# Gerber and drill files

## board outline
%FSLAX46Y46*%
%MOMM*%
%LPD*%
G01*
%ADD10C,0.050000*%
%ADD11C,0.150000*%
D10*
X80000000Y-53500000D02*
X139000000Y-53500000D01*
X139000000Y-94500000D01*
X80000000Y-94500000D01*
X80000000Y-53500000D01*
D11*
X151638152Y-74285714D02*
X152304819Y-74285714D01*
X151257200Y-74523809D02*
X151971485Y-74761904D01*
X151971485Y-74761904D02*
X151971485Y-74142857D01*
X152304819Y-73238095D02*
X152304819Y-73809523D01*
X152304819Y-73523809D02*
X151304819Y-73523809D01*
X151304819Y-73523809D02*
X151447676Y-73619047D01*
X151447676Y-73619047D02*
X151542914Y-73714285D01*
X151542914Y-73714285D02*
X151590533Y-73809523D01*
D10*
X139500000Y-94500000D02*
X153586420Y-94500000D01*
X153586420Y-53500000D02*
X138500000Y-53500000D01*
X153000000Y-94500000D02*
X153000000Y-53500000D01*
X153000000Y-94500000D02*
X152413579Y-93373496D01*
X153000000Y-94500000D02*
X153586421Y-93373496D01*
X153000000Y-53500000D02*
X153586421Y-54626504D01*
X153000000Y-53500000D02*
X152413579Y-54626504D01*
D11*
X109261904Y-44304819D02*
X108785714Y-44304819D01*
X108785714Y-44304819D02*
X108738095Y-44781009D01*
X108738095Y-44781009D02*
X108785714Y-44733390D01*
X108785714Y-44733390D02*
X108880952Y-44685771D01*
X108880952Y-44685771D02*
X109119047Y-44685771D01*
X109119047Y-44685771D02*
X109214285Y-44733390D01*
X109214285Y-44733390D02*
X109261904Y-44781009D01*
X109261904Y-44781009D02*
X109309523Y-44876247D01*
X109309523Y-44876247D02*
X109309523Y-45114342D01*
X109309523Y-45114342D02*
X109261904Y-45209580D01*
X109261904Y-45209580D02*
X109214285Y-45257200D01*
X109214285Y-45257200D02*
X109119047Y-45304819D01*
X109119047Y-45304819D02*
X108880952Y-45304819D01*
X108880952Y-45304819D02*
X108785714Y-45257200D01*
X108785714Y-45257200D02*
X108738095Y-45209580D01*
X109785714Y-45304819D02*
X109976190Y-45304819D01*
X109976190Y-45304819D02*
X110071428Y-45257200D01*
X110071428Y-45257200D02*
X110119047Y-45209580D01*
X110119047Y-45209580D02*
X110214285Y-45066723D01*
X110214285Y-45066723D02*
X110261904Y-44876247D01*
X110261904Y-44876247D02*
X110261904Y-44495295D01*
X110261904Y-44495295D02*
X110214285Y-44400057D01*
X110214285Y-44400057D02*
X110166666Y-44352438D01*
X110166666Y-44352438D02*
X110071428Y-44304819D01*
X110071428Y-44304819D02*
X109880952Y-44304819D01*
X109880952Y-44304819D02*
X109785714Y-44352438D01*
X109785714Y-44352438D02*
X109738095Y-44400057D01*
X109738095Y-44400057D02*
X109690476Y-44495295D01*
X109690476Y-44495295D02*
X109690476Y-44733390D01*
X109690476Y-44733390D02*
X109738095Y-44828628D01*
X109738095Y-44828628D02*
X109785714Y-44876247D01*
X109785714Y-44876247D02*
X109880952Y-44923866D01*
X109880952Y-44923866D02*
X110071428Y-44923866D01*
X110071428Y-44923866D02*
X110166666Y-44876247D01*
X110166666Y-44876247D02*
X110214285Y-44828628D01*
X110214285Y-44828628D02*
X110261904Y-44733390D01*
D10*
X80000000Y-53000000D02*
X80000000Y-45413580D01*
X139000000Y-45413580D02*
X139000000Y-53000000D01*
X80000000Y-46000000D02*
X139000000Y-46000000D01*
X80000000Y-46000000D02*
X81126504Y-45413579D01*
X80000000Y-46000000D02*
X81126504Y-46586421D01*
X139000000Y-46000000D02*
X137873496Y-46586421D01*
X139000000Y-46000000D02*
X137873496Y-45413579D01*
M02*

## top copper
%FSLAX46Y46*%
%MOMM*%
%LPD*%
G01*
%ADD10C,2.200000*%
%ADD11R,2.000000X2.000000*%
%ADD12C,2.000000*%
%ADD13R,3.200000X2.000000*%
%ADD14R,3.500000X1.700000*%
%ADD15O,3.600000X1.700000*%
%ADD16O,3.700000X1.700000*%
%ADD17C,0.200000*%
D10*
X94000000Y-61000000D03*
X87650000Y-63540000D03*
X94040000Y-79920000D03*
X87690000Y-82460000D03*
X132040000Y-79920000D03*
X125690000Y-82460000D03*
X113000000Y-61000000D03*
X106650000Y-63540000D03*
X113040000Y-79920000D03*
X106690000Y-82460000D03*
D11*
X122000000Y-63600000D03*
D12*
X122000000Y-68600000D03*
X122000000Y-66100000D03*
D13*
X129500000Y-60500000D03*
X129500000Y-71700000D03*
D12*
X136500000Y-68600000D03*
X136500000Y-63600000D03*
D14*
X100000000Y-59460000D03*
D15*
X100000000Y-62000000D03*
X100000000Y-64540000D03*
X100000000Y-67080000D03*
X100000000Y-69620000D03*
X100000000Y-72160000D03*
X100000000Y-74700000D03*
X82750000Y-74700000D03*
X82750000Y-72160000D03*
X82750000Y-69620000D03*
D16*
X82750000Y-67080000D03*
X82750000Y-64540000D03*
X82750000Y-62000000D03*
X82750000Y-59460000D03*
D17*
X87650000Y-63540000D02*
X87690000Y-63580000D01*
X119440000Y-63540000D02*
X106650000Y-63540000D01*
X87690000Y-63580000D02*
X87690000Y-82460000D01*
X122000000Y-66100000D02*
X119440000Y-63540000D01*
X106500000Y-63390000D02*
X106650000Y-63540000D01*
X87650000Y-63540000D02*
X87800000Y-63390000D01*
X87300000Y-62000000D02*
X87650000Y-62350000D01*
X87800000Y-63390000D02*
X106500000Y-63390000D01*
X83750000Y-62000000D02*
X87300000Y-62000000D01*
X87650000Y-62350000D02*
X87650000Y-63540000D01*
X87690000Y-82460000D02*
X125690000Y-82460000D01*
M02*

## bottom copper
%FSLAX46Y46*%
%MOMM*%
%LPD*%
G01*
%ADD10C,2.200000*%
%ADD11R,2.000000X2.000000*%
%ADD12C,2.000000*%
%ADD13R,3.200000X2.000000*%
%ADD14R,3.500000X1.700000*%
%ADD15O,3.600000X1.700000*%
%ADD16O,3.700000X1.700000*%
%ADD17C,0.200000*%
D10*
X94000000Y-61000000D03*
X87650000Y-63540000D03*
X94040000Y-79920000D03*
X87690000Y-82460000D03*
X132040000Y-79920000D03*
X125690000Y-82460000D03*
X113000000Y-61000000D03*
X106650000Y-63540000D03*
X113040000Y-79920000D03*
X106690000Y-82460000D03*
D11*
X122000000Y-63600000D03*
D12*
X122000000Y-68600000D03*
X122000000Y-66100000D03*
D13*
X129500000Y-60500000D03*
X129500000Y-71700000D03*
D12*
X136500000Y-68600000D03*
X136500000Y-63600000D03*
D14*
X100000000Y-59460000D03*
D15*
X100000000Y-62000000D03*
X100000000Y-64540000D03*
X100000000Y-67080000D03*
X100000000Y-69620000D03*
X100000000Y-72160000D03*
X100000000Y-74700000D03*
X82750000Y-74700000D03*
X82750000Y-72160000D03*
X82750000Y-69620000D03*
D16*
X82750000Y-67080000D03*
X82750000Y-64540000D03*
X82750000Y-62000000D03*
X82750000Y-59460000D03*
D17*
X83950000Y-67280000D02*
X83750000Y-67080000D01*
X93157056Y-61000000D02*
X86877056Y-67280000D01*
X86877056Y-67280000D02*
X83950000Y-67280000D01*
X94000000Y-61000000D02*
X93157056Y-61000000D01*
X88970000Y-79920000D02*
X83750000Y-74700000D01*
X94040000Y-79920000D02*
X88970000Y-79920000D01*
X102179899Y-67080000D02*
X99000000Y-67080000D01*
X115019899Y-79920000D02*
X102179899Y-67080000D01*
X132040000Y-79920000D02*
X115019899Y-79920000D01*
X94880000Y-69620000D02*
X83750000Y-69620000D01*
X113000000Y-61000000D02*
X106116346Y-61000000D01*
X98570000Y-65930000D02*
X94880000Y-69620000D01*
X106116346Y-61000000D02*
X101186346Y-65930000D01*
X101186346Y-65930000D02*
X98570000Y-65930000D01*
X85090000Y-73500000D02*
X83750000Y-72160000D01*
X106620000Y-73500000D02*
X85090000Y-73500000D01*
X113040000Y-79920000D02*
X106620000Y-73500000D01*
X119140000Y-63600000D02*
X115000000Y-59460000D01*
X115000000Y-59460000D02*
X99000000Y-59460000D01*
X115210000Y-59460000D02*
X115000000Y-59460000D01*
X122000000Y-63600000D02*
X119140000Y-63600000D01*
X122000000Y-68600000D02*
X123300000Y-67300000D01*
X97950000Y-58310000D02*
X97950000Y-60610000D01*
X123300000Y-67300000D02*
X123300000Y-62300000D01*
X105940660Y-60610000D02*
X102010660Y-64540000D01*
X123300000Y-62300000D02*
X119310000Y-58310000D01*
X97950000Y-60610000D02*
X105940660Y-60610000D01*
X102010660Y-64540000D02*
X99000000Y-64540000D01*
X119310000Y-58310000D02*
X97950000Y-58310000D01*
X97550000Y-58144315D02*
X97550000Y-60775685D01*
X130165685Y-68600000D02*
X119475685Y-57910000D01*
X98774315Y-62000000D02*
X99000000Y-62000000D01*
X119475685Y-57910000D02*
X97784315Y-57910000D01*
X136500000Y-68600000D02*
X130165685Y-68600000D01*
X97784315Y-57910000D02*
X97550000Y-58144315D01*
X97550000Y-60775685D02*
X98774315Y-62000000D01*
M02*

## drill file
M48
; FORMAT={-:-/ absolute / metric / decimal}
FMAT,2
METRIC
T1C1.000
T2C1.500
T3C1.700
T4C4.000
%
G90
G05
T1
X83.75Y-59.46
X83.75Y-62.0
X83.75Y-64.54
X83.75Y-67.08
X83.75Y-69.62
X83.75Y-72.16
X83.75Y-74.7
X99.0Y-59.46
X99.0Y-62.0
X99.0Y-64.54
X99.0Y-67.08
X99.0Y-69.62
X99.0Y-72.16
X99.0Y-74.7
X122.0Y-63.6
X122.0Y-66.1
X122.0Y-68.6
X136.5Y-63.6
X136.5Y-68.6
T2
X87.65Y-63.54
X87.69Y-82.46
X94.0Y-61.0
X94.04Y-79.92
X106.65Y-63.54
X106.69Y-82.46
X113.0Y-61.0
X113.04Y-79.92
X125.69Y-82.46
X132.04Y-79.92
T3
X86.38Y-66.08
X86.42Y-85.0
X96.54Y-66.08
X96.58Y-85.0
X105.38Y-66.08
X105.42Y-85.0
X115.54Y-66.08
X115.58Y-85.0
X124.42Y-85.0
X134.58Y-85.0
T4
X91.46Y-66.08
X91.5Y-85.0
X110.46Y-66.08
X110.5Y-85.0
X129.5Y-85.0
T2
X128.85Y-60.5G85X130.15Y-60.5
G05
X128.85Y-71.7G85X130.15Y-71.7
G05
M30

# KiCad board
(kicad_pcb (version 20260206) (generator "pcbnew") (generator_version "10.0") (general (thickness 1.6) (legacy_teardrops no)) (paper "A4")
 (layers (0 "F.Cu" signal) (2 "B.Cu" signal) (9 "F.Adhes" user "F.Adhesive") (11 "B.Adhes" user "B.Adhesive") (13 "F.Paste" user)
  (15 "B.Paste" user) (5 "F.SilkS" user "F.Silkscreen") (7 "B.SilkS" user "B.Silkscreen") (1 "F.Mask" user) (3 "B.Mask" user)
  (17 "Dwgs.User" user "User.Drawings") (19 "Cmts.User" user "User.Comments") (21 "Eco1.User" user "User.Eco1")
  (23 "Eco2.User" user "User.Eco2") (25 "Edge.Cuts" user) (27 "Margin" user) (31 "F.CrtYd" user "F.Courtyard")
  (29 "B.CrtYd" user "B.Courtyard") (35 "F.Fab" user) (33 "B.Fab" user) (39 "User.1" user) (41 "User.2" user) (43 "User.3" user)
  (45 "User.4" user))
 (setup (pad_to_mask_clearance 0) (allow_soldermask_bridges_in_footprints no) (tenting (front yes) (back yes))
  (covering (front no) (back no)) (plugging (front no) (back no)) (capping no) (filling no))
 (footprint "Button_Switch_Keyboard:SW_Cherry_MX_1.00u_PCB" (layer "F.Cu") (at 94 61)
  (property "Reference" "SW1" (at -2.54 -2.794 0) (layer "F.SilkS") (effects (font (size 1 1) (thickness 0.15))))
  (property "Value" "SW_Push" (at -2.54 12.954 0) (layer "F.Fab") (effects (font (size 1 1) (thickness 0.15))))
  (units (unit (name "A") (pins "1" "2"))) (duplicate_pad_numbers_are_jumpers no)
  (pad "" np_thru_hole circle (at -7.62 5.08) (size 1.7 1.7) (drill 1.7) (layers "*.Cu" "*.Mask"))
  (pad "" np_thru_hole circle (at -2.54 5.08) (size 4 4) (drill 4) (layers "*.Cu" "*.Mask"))
  (pad "" np_thru_hole circle (at 2.54 5.08) (size 1.7 1.7) (drill 1.7) (layers "*.Cu" "*.Mask"))
  (pad "1" thru_hole circle (at 0 0) (size 2.2 2.2) (drill 1.5) (layers "*.Cu" "*.Mask") (remove_unused_layers no)
   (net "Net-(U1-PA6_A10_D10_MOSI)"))
  (pad "2" thru_hole circle (at -6.35 2.54) (size 2.2 2.2) (drill 1.5) (layers "*.Cu" "*.Mask") (remove_unused_layers no) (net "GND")))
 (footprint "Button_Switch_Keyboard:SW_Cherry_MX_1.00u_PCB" (layer "F.Cu") (at 94.04 79.92)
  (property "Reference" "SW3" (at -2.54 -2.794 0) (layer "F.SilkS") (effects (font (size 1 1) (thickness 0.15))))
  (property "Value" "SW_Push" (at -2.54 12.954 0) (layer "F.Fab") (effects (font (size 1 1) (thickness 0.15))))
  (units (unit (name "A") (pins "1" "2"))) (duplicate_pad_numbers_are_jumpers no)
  (pad "" np_thru_hole circle (at -7.62 5.08) (size 1.7 1.7) (drill 1.7) (layers "*.Cu" "*.Mask"))
  (pad "" np_thru_hole circle (at -2.54 5.08) (size 4 4) (drill 4) (layers "*.Cu" "*.Mask"))
  (pad "" np_thru_hole circle (at 2.54 5.08) (size 1.7 1.7) (drill 1.7) (layers "*.Cu" "*.Mask"))
  (pad "1" thru_hole circle (at 0 0) (size 2.2 2.2) (drill 1.5) (layers "*.Cu" "*.Mask") (remove_unused_layers no)
   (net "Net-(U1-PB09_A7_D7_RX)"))
  (pad "2" thru_hole circle (at -6.35 2.54) (size 2.2 2.2) (drill 1.5) (layers "*.Cu" "*.Mask") (remove_unused_layers no) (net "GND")))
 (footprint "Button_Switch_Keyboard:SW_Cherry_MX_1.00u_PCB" (layer "F.Cu") (at 132.04 79.92)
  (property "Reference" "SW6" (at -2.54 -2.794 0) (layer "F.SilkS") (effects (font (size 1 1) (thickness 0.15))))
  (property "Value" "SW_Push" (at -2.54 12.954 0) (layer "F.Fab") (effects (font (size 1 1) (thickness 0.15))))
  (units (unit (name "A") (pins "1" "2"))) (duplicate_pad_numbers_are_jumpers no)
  (pad "" np_thru_hole circle (at -7.62 5.08) (size 1.7 1.7) (drill 1.7) (layers "*.Cu" "*.Mask"))
  (pad "" np_thru_hole circle (at -2.54 5.08) (size 4 4) (drill 4) (layers "*.Cu" "*.Mask"))
  (pad "" np_thru_hole circle (at 2.54 5.08) (size 1.7 1.7) (drill 1.7) (layers "*.Cu" "*.Mask"))
  (pad "1" thru_hole circle (at 0 0) (size 2.2 2.2) (drill 1.5) (layers "*.Cu" "*.Mask") (remove_unused_layers no)
   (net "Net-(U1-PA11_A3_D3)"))
  (pad "2" thru_hole circle (at -6.35 2.54) (size 2.2 2.2) (drill 1.5) (layers "*.Cu" "*.Mask") (remove_unused_layers no) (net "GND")))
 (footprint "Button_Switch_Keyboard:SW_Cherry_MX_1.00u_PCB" (layer "F.Cu") (at 113 61)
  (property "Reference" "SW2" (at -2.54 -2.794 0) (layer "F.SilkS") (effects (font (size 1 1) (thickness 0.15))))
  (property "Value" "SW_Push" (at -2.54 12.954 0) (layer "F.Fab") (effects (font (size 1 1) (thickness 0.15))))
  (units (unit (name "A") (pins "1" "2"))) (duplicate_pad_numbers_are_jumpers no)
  (pad "" np_thru_hole circle (at -7.62 5.08) (size 1.7 1.7) (drill 1.7) (layers "*.Cu" "*.Mask"))
  (pad "" np_thru_hole circle (at -2.54 5.08) (size 4 4) (drill 4) (layers "*.Cu" "*.Mask"))
  (pad "" np_thru_hole circle (at 2.54 5.08) (size 1.7 1.7) (drill 1.7) (layers "*.Cu" "*.Mask"))
  (pad "1" thru_hole circle (at 0 0) (size 2.2 2.2) (drill 1.5) (layers "*.Cu" "*.Mask") (remove_unused_layers no)
   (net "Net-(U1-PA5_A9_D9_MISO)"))
  (pad "2" thru_hole circle (at -6.35 2.54) (size 2.2 2.2) (drill 1.5) (layers "*.Cu" "*.Mask") (remove_unused_layers no) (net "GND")))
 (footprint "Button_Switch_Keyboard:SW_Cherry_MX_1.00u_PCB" (layer "F.Cu") (at 113.04 79.92)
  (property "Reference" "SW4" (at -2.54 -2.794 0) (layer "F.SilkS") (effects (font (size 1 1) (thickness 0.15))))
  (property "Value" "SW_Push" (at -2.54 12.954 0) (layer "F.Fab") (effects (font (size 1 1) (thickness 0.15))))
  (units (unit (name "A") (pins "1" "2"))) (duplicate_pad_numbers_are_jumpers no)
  (pad "" np_thru_hole circle (at -7.62 5.08) (size 1.7 1.7) (drill 1.7) (layers "*.Cu" "*.Mask"))
  (pad "" np_thru_hole circle (at -2.54 5.08) (size 4 4) (drill 4) (layers "*.Cu" "*.Mask"))
  (pad "" np_thru_hole circle (at 2.54 5.08) (size 1.7 1.7) (drill 1.7) (layers "*.Cu" "*.Mask"))
  (pad "1" thru_hole circle (at 0 0) (size 2.2 2.2) (drill 1.5) (layers "*.Cu" "*.Mask") (remove_unused_layers no)
   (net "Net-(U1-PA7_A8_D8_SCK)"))
  (pad "2" thru_hole circle (at -6.35 2.54) (size 2.2 2.2) (drill 1.5) (layers "*.Cu" "*.Mask") (remove_unused_layers no) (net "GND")))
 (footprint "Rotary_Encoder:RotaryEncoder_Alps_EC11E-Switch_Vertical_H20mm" (layer "F.Cu") (at 122 63.6)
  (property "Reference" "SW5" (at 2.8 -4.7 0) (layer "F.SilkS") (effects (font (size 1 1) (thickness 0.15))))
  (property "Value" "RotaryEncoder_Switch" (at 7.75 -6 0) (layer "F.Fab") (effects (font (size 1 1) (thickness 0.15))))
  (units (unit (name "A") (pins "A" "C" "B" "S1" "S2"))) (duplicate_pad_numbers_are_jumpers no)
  (pad "A" thru_hole rect (at 0 0) (size 2 2) (drill 1) (layers "*.Cu" "*.Mask") (remove_unused_layers no) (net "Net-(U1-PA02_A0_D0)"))
  (pad "B" thru_hole circle (at 0 5) (size 2 2) (drill 1) (layers "*.Cu" "*.Mask") (remove_unused_layers no) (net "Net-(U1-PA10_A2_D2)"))
  (pad "C" thru_hole circle (at 0 2.5) (size 2 2) (drill 1) (layers "*.Cu" "*.Mask") (remove_unused_layers no) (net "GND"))
  (pad "MP" thru_hole rect (at 7.5 -3.1) (size 3.2 2) (drill oval 2.8 1.5) (layers "*.Cu" "*.Mask") (remove_unused_layers no))
  (pad "MP" thru_hole rect (at 7.5 8.1) (size 3.2 2) (drill oval 2.8 1.5) (layers "*.Cu" "*.Mask") (remove_unused_layers no))
  (pad "S1" thru_hole circle (at 14.5 5) (size 2 2) (drill 1) (layers "*.Cu" "*.Mask") (remove_unused_layers no) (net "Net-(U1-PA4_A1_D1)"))
  (pad "S2" thru_hole circle (at 14.5 0) (size 2 2) (drill 1) (layers "*.Cu" "*.Mask") (remove_unused_layers no)
   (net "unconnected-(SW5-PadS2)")))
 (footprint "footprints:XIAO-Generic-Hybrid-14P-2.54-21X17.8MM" (layer "B.Cu") (at 91.375 67.08 180)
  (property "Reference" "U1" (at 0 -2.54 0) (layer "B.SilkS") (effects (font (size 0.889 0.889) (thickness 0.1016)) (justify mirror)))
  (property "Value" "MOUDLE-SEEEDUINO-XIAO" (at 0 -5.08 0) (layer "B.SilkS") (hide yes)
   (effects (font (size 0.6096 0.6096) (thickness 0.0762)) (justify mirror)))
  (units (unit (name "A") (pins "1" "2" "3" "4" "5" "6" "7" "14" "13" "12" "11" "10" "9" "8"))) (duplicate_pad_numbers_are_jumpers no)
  (pad "1" thru_hole rect (at -7.625 7.62 180) (size 3.5 1.7) (drill 1 (offset -1 0)) (layers "*.Cu" "*.Mask") (remove_unused_layers no)
   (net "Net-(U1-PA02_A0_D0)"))
  (pad "2" thru_hole oval (at -7.625 5.08 180) (size 3.6 1.7) (drill 1 (offset -1 0)) (layers "*.Cu" "*.Mask") (remove_unused_layers no)
   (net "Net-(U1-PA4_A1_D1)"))
  (pad "3" thru_hole oval (at -7.625 2.54 180) (size 3.6 1.7) (drill 1 (offset -1 0)) (layers "*.Cu" "*.Mask") (remove_unused_layers no)
   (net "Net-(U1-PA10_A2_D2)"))
  (pad "4" thru_hole oval (at -7.625 0 180) (size 3.6 1.7) (drill 1 (offset -1 0)) (layers "*.Cu" "*.Mask") (remove_unused_layers no)
   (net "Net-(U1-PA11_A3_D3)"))
  (pad "5" thru_hole oval (at -7.625 -2.54 180) (size 3.6 1.7) (drill 1 (offset -1 0)) (layers "*.Cu" "*.Mask") (remove_unused_layers no)
   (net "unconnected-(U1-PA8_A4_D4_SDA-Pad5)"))
  (pad "6" thru_hole oval (at -7.625 -5.08) (size 3.6 1.7) (drill 1 (offset 1 0)) (layers "*.Cu" "*.Mask") (remove_unused_layers no)
   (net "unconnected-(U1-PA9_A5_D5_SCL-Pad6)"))
  (pad "7" thru_hole oval (at -7.625 -7.62 180) (size 3.6 1.7) (drill 1 (offset -1 0)) (layers "*.Cu" "*.Mask") (remove_unused_layers no)
   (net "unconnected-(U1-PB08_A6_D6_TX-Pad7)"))
  (pad "8" thru_hole oval (at 7.625 -7.62 180) (size 3.6 1.7) (drill 1 (offset 1 0)) (layers "*.Cu" "*.Mask") (remove_unused_layers no)
   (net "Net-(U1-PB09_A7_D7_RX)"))
  (pad "9" thru_hole oval (at 7.625 -5.08 180) (size 3.6 1.7) (drill 1 (offset 1 0)) (layers "*.Cu" "*.Mask") (remove_unused_layers no)
   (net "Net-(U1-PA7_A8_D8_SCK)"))
  (pad "10" thru_hole oval (at 7.625 -2.54 180) (size 3.6 1.7) (drill 1 (offset 1 0)) (layers "*.Cu" "*.Mask") (remove_unused_layers no)
   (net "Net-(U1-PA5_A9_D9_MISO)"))
  (pad "11" thru_hole oval (at 7.625 0 180) (size 3.7 1.7) (drill 1 (offset 1 0)) (layers "*.Cu" "*.Mask") (remove_unused_layers no)
   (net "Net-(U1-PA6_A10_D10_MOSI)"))
  (pad "12" thru_hole oval (at 7.625 2.54 180) (size 3.7 1.7) (drill 1 (offset 1 0)) (layers "*.Cu" "*.Mask") (remove_unused_layers no)
   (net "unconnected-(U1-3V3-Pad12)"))
  (pad "13" thru_hole oval (at 7.625 5.08 180) (size 3.7 1.7) (drill 1 (offset 1 0)) (layers "*.Cu" "*.Mask") (remove_unused_layers no)
   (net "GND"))
  (pad "14" thru_hole oval (at 7.625 7.62 180) (size 3.7 1.7) (drill 1 (offset 1 0)) (layers "*.Cu" "*.Mask") (remove_unused_layers no)
   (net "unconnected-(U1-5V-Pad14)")))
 (gr_rect (start 80 53.5) (end 139 94.5) (stroke (width 0.05) (type default)) (fill no) (layer "Edge.Cuts"))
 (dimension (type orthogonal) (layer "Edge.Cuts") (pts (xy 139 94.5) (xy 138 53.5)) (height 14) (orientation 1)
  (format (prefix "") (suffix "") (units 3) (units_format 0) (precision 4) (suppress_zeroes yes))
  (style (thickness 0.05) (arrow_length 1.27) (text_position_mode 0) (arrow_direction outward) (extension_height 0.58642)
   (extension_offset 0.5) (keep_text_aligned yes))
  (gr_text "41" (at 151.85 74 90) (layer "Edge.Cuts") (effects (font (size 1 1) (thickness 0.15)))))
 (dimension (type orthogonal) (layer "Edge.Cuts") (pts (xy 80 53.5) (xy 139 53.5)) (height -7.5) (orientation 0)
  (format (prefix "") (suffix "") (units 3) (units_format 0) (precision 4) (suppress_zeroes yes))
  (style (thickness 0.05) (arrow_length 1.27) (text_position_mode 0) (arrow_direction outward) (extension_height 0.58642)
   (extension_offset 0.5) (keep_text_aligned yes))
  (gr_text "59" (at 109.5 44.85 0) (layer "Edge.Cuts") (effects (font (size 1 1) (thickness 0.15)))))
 (segment (start 83.95 67.28) (end 83.75 67.08) (width 0.2) (layer "B.Cu") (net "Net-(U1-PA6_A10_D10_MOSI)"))
 (segment (start 93.157056 61) (end 86.877056 67.28) (width 0.2) (layer "B.Cu") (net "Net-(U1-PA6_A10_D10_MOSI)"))
 (segment (start 86.877056 67.28) (end 83.95 67.28) (width 0.2) (layer "B.Cu") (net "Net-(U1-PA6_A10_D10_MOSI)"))
 (segment (start 94 61) (end 93.157056 61) (width 0.2) (layer "B.Cu") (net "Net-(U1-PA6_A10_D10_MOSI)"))
 (segment (start 87.65 63.54) (end 87.69 63.58) (width 0.2) (layer "F.Cu") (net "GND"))
 (segment (start 119.44 63.54) (end 106.65 63.54) (width 0.2) (layer "F.Cu") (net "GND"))
 (segment (start 87.69 63.58) (end 87.69 82.46) (width 0.2) (layer "F.Cu") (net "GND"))
 (segment (start 122 66.1) (end 119.44 63.54) (width 0.2) (layer "F.Cu") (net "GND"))
 (segment (start 106.5 63.39) (end 106.65 63.54) (width 0.2) (layer "F.Cu") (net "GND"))
 (segment (start 87.65 63.54) (end 87.8 63.39) (width 0.2) (layer "F.Cu") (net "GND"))
 (segment (start 87.3 62) (end 87.65 62.35) (width 0.2) (layer "F.Cu") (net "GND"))
 (segment (start 87.8 63.39) (end 106.5 63.39) (width 0.2) (layer "F.Cu") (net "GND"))
 (segment (start 83.75 62) (end 87.3 62) (width 0.2) (layer "F.Cu") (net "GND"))
 (segment (start 87.65 62.35) (end 87.65 63.54) (width 0.2) (layer "F.Cu") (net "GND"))
 (segment (start 87.69 82.46) (end 125.69 82.46) (width 0.2) (layer "F.Cu") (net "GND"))
 (segment (start 88.97 79.92) (end 83.75 74.7) (width 0.2) (layer "B.Cu") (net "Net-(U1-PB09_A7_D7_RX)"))
 (segment (start 94.04 79.92) (end 88.97 79.92) (width 0.2) (layer "B.Cu") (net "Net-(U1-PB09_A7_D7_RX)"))
 (segment (start 102.179899 67.08) (end 99 67.08) (width 0.2) (layer "B.Cu") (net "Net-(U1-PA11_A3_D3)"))
 (segment (start 115.019899 79.92) (end 102.179899 67.08) (width 0.2) (layer "B.Cu") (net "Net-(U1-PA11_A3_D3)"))
 (segment (start 132.04 79.92) (end 115.019899 79.92) (width 0.2) (layer "B.Cu") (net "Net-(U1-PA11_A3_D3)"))
 (segment (start 94.88 69.62) (end 83.75 69.62) (width 0.2) (layer "B.Cu") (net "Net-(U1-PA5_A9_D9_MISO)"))
 (segment (start 113 61) (end 106.116346 61) (width 0.2) (layer "B.Cu") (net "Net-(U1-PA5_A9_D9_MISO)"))
 (segment (start 98.57 65.93) (end 94.88 69.62) (width 0.2) (layer "B.Cu") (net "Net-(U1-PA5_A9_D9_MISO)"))
 (segment (start 106.116346 61) (end 101.186346 65.93) (width 0.2) (layer "B.Cu") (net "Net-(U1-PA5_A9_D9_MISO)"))
 (segment (start 101.186346 65.93) (end 98.57 65.93) (width 0.2) (layer "B.Cu") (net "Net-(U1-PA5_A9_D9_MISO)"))
 (segment (start 85.09 73.5) (end 83.75 72.16) (width 0.2) (layer "B.Cu") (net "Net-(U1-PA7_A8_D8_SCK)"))
 (segment (start 106.62 73.5) (end 85.09 73.5) (width 0.2) (layer "B.Cu") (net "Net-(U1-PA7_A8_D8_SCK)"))
 (segment (start 113.04 79.92) (end 106.62 73.5) (width 0.2) (layer "B.Cu") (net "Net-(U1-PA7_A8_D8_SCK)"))
 (segment (start 119.14 63.6) (end 115 59.46) (width 0.2) (layer "B.Cu") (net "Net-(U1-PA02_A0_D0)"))
 (segment (start 115 59.46) (end 99 59.46) (width 0.2) (layer "B.Cu") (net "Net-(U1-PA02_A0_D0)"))
 (segment (start 115.21 59.46) (end 115 59.46) (width 0.2) (layer "B.Cu") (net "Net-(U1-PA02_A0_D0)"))
 (segment (start 122 63.6) (end 119.14 63.6) (width 0.2) (layer "B.Cu") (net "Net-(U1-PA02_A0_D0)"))
 (segment (start 122 68.6) (end 123.3 67.3) (width 0.2) (layer "B.Cu") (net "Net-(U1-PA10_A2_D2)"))
 (segment (start 97.95 58.31) (end 97.95 60.61) (width 0.2) (layer "B.Cu") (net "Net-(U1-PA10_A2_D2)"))
 (segment (start 123.3 67.3) (end 123.3 62.3) (width 0.2) (layer "B.Cu") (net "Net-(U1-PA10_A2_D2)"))
 (segment (start 105.94066 60.61) (end 102.01066 64.54) (width 0.2) (layer "B.Cu") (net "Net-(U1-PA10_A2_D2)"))
 (segment (start 123.3 62.3) (end 119.31 58.31) (width 0.2) (layer "B.Cu") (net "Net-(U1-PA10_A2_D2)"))
 (segment (start 97.95 60.61) (end 105.94066 60.61) (width 0.2) (layer "B.Cu") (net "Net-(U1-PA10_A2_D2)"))
 (segment (start 102.01066 64.54) (end 99 64.54) (width 0.2) (layer "B.Cu") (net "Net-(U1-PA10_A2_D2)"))
 (segment (start 119.31 58.31) (end 97.95 58.31) (width 0.2) (layer "B.Cu") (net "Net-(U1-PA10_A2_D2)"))
 (segment (start 97.55 58.144315) (end 97.55 60.775685) (width 0.2) (layer "B.Cu") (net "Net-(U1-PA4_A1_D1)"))
 (segment (start 130.165685 68.6) (end 119.475685 57.91) (width 0.2) (layer "B.Cu") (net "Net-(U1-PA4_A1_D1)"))
 (segment (start 98.774315 62) (end 99 62) (width 0.2) (layer "B.Cu") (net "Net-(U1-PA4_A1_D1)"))
 (segment (start 119.475685 57.91) (end 97.784315 57.91) (width 0.2) (layer "B.Cu") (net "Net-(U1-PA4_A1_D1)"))
 (segment (start 136.5 68.6) (end 130.165685 68.6) (width 0.2) (layer "B.Cu") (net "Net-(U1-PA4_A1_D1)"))
 (segment (start 97.784315 57.91) (end 97.55 58.144315) (width 0.2) (layer "B.Cu") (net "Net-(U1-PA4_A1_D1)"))
 (segment (start 97.55 60.775685) (end 98.774315 62) (width 0.2) (layer "B.Cu") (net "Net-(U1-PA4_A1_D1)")))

